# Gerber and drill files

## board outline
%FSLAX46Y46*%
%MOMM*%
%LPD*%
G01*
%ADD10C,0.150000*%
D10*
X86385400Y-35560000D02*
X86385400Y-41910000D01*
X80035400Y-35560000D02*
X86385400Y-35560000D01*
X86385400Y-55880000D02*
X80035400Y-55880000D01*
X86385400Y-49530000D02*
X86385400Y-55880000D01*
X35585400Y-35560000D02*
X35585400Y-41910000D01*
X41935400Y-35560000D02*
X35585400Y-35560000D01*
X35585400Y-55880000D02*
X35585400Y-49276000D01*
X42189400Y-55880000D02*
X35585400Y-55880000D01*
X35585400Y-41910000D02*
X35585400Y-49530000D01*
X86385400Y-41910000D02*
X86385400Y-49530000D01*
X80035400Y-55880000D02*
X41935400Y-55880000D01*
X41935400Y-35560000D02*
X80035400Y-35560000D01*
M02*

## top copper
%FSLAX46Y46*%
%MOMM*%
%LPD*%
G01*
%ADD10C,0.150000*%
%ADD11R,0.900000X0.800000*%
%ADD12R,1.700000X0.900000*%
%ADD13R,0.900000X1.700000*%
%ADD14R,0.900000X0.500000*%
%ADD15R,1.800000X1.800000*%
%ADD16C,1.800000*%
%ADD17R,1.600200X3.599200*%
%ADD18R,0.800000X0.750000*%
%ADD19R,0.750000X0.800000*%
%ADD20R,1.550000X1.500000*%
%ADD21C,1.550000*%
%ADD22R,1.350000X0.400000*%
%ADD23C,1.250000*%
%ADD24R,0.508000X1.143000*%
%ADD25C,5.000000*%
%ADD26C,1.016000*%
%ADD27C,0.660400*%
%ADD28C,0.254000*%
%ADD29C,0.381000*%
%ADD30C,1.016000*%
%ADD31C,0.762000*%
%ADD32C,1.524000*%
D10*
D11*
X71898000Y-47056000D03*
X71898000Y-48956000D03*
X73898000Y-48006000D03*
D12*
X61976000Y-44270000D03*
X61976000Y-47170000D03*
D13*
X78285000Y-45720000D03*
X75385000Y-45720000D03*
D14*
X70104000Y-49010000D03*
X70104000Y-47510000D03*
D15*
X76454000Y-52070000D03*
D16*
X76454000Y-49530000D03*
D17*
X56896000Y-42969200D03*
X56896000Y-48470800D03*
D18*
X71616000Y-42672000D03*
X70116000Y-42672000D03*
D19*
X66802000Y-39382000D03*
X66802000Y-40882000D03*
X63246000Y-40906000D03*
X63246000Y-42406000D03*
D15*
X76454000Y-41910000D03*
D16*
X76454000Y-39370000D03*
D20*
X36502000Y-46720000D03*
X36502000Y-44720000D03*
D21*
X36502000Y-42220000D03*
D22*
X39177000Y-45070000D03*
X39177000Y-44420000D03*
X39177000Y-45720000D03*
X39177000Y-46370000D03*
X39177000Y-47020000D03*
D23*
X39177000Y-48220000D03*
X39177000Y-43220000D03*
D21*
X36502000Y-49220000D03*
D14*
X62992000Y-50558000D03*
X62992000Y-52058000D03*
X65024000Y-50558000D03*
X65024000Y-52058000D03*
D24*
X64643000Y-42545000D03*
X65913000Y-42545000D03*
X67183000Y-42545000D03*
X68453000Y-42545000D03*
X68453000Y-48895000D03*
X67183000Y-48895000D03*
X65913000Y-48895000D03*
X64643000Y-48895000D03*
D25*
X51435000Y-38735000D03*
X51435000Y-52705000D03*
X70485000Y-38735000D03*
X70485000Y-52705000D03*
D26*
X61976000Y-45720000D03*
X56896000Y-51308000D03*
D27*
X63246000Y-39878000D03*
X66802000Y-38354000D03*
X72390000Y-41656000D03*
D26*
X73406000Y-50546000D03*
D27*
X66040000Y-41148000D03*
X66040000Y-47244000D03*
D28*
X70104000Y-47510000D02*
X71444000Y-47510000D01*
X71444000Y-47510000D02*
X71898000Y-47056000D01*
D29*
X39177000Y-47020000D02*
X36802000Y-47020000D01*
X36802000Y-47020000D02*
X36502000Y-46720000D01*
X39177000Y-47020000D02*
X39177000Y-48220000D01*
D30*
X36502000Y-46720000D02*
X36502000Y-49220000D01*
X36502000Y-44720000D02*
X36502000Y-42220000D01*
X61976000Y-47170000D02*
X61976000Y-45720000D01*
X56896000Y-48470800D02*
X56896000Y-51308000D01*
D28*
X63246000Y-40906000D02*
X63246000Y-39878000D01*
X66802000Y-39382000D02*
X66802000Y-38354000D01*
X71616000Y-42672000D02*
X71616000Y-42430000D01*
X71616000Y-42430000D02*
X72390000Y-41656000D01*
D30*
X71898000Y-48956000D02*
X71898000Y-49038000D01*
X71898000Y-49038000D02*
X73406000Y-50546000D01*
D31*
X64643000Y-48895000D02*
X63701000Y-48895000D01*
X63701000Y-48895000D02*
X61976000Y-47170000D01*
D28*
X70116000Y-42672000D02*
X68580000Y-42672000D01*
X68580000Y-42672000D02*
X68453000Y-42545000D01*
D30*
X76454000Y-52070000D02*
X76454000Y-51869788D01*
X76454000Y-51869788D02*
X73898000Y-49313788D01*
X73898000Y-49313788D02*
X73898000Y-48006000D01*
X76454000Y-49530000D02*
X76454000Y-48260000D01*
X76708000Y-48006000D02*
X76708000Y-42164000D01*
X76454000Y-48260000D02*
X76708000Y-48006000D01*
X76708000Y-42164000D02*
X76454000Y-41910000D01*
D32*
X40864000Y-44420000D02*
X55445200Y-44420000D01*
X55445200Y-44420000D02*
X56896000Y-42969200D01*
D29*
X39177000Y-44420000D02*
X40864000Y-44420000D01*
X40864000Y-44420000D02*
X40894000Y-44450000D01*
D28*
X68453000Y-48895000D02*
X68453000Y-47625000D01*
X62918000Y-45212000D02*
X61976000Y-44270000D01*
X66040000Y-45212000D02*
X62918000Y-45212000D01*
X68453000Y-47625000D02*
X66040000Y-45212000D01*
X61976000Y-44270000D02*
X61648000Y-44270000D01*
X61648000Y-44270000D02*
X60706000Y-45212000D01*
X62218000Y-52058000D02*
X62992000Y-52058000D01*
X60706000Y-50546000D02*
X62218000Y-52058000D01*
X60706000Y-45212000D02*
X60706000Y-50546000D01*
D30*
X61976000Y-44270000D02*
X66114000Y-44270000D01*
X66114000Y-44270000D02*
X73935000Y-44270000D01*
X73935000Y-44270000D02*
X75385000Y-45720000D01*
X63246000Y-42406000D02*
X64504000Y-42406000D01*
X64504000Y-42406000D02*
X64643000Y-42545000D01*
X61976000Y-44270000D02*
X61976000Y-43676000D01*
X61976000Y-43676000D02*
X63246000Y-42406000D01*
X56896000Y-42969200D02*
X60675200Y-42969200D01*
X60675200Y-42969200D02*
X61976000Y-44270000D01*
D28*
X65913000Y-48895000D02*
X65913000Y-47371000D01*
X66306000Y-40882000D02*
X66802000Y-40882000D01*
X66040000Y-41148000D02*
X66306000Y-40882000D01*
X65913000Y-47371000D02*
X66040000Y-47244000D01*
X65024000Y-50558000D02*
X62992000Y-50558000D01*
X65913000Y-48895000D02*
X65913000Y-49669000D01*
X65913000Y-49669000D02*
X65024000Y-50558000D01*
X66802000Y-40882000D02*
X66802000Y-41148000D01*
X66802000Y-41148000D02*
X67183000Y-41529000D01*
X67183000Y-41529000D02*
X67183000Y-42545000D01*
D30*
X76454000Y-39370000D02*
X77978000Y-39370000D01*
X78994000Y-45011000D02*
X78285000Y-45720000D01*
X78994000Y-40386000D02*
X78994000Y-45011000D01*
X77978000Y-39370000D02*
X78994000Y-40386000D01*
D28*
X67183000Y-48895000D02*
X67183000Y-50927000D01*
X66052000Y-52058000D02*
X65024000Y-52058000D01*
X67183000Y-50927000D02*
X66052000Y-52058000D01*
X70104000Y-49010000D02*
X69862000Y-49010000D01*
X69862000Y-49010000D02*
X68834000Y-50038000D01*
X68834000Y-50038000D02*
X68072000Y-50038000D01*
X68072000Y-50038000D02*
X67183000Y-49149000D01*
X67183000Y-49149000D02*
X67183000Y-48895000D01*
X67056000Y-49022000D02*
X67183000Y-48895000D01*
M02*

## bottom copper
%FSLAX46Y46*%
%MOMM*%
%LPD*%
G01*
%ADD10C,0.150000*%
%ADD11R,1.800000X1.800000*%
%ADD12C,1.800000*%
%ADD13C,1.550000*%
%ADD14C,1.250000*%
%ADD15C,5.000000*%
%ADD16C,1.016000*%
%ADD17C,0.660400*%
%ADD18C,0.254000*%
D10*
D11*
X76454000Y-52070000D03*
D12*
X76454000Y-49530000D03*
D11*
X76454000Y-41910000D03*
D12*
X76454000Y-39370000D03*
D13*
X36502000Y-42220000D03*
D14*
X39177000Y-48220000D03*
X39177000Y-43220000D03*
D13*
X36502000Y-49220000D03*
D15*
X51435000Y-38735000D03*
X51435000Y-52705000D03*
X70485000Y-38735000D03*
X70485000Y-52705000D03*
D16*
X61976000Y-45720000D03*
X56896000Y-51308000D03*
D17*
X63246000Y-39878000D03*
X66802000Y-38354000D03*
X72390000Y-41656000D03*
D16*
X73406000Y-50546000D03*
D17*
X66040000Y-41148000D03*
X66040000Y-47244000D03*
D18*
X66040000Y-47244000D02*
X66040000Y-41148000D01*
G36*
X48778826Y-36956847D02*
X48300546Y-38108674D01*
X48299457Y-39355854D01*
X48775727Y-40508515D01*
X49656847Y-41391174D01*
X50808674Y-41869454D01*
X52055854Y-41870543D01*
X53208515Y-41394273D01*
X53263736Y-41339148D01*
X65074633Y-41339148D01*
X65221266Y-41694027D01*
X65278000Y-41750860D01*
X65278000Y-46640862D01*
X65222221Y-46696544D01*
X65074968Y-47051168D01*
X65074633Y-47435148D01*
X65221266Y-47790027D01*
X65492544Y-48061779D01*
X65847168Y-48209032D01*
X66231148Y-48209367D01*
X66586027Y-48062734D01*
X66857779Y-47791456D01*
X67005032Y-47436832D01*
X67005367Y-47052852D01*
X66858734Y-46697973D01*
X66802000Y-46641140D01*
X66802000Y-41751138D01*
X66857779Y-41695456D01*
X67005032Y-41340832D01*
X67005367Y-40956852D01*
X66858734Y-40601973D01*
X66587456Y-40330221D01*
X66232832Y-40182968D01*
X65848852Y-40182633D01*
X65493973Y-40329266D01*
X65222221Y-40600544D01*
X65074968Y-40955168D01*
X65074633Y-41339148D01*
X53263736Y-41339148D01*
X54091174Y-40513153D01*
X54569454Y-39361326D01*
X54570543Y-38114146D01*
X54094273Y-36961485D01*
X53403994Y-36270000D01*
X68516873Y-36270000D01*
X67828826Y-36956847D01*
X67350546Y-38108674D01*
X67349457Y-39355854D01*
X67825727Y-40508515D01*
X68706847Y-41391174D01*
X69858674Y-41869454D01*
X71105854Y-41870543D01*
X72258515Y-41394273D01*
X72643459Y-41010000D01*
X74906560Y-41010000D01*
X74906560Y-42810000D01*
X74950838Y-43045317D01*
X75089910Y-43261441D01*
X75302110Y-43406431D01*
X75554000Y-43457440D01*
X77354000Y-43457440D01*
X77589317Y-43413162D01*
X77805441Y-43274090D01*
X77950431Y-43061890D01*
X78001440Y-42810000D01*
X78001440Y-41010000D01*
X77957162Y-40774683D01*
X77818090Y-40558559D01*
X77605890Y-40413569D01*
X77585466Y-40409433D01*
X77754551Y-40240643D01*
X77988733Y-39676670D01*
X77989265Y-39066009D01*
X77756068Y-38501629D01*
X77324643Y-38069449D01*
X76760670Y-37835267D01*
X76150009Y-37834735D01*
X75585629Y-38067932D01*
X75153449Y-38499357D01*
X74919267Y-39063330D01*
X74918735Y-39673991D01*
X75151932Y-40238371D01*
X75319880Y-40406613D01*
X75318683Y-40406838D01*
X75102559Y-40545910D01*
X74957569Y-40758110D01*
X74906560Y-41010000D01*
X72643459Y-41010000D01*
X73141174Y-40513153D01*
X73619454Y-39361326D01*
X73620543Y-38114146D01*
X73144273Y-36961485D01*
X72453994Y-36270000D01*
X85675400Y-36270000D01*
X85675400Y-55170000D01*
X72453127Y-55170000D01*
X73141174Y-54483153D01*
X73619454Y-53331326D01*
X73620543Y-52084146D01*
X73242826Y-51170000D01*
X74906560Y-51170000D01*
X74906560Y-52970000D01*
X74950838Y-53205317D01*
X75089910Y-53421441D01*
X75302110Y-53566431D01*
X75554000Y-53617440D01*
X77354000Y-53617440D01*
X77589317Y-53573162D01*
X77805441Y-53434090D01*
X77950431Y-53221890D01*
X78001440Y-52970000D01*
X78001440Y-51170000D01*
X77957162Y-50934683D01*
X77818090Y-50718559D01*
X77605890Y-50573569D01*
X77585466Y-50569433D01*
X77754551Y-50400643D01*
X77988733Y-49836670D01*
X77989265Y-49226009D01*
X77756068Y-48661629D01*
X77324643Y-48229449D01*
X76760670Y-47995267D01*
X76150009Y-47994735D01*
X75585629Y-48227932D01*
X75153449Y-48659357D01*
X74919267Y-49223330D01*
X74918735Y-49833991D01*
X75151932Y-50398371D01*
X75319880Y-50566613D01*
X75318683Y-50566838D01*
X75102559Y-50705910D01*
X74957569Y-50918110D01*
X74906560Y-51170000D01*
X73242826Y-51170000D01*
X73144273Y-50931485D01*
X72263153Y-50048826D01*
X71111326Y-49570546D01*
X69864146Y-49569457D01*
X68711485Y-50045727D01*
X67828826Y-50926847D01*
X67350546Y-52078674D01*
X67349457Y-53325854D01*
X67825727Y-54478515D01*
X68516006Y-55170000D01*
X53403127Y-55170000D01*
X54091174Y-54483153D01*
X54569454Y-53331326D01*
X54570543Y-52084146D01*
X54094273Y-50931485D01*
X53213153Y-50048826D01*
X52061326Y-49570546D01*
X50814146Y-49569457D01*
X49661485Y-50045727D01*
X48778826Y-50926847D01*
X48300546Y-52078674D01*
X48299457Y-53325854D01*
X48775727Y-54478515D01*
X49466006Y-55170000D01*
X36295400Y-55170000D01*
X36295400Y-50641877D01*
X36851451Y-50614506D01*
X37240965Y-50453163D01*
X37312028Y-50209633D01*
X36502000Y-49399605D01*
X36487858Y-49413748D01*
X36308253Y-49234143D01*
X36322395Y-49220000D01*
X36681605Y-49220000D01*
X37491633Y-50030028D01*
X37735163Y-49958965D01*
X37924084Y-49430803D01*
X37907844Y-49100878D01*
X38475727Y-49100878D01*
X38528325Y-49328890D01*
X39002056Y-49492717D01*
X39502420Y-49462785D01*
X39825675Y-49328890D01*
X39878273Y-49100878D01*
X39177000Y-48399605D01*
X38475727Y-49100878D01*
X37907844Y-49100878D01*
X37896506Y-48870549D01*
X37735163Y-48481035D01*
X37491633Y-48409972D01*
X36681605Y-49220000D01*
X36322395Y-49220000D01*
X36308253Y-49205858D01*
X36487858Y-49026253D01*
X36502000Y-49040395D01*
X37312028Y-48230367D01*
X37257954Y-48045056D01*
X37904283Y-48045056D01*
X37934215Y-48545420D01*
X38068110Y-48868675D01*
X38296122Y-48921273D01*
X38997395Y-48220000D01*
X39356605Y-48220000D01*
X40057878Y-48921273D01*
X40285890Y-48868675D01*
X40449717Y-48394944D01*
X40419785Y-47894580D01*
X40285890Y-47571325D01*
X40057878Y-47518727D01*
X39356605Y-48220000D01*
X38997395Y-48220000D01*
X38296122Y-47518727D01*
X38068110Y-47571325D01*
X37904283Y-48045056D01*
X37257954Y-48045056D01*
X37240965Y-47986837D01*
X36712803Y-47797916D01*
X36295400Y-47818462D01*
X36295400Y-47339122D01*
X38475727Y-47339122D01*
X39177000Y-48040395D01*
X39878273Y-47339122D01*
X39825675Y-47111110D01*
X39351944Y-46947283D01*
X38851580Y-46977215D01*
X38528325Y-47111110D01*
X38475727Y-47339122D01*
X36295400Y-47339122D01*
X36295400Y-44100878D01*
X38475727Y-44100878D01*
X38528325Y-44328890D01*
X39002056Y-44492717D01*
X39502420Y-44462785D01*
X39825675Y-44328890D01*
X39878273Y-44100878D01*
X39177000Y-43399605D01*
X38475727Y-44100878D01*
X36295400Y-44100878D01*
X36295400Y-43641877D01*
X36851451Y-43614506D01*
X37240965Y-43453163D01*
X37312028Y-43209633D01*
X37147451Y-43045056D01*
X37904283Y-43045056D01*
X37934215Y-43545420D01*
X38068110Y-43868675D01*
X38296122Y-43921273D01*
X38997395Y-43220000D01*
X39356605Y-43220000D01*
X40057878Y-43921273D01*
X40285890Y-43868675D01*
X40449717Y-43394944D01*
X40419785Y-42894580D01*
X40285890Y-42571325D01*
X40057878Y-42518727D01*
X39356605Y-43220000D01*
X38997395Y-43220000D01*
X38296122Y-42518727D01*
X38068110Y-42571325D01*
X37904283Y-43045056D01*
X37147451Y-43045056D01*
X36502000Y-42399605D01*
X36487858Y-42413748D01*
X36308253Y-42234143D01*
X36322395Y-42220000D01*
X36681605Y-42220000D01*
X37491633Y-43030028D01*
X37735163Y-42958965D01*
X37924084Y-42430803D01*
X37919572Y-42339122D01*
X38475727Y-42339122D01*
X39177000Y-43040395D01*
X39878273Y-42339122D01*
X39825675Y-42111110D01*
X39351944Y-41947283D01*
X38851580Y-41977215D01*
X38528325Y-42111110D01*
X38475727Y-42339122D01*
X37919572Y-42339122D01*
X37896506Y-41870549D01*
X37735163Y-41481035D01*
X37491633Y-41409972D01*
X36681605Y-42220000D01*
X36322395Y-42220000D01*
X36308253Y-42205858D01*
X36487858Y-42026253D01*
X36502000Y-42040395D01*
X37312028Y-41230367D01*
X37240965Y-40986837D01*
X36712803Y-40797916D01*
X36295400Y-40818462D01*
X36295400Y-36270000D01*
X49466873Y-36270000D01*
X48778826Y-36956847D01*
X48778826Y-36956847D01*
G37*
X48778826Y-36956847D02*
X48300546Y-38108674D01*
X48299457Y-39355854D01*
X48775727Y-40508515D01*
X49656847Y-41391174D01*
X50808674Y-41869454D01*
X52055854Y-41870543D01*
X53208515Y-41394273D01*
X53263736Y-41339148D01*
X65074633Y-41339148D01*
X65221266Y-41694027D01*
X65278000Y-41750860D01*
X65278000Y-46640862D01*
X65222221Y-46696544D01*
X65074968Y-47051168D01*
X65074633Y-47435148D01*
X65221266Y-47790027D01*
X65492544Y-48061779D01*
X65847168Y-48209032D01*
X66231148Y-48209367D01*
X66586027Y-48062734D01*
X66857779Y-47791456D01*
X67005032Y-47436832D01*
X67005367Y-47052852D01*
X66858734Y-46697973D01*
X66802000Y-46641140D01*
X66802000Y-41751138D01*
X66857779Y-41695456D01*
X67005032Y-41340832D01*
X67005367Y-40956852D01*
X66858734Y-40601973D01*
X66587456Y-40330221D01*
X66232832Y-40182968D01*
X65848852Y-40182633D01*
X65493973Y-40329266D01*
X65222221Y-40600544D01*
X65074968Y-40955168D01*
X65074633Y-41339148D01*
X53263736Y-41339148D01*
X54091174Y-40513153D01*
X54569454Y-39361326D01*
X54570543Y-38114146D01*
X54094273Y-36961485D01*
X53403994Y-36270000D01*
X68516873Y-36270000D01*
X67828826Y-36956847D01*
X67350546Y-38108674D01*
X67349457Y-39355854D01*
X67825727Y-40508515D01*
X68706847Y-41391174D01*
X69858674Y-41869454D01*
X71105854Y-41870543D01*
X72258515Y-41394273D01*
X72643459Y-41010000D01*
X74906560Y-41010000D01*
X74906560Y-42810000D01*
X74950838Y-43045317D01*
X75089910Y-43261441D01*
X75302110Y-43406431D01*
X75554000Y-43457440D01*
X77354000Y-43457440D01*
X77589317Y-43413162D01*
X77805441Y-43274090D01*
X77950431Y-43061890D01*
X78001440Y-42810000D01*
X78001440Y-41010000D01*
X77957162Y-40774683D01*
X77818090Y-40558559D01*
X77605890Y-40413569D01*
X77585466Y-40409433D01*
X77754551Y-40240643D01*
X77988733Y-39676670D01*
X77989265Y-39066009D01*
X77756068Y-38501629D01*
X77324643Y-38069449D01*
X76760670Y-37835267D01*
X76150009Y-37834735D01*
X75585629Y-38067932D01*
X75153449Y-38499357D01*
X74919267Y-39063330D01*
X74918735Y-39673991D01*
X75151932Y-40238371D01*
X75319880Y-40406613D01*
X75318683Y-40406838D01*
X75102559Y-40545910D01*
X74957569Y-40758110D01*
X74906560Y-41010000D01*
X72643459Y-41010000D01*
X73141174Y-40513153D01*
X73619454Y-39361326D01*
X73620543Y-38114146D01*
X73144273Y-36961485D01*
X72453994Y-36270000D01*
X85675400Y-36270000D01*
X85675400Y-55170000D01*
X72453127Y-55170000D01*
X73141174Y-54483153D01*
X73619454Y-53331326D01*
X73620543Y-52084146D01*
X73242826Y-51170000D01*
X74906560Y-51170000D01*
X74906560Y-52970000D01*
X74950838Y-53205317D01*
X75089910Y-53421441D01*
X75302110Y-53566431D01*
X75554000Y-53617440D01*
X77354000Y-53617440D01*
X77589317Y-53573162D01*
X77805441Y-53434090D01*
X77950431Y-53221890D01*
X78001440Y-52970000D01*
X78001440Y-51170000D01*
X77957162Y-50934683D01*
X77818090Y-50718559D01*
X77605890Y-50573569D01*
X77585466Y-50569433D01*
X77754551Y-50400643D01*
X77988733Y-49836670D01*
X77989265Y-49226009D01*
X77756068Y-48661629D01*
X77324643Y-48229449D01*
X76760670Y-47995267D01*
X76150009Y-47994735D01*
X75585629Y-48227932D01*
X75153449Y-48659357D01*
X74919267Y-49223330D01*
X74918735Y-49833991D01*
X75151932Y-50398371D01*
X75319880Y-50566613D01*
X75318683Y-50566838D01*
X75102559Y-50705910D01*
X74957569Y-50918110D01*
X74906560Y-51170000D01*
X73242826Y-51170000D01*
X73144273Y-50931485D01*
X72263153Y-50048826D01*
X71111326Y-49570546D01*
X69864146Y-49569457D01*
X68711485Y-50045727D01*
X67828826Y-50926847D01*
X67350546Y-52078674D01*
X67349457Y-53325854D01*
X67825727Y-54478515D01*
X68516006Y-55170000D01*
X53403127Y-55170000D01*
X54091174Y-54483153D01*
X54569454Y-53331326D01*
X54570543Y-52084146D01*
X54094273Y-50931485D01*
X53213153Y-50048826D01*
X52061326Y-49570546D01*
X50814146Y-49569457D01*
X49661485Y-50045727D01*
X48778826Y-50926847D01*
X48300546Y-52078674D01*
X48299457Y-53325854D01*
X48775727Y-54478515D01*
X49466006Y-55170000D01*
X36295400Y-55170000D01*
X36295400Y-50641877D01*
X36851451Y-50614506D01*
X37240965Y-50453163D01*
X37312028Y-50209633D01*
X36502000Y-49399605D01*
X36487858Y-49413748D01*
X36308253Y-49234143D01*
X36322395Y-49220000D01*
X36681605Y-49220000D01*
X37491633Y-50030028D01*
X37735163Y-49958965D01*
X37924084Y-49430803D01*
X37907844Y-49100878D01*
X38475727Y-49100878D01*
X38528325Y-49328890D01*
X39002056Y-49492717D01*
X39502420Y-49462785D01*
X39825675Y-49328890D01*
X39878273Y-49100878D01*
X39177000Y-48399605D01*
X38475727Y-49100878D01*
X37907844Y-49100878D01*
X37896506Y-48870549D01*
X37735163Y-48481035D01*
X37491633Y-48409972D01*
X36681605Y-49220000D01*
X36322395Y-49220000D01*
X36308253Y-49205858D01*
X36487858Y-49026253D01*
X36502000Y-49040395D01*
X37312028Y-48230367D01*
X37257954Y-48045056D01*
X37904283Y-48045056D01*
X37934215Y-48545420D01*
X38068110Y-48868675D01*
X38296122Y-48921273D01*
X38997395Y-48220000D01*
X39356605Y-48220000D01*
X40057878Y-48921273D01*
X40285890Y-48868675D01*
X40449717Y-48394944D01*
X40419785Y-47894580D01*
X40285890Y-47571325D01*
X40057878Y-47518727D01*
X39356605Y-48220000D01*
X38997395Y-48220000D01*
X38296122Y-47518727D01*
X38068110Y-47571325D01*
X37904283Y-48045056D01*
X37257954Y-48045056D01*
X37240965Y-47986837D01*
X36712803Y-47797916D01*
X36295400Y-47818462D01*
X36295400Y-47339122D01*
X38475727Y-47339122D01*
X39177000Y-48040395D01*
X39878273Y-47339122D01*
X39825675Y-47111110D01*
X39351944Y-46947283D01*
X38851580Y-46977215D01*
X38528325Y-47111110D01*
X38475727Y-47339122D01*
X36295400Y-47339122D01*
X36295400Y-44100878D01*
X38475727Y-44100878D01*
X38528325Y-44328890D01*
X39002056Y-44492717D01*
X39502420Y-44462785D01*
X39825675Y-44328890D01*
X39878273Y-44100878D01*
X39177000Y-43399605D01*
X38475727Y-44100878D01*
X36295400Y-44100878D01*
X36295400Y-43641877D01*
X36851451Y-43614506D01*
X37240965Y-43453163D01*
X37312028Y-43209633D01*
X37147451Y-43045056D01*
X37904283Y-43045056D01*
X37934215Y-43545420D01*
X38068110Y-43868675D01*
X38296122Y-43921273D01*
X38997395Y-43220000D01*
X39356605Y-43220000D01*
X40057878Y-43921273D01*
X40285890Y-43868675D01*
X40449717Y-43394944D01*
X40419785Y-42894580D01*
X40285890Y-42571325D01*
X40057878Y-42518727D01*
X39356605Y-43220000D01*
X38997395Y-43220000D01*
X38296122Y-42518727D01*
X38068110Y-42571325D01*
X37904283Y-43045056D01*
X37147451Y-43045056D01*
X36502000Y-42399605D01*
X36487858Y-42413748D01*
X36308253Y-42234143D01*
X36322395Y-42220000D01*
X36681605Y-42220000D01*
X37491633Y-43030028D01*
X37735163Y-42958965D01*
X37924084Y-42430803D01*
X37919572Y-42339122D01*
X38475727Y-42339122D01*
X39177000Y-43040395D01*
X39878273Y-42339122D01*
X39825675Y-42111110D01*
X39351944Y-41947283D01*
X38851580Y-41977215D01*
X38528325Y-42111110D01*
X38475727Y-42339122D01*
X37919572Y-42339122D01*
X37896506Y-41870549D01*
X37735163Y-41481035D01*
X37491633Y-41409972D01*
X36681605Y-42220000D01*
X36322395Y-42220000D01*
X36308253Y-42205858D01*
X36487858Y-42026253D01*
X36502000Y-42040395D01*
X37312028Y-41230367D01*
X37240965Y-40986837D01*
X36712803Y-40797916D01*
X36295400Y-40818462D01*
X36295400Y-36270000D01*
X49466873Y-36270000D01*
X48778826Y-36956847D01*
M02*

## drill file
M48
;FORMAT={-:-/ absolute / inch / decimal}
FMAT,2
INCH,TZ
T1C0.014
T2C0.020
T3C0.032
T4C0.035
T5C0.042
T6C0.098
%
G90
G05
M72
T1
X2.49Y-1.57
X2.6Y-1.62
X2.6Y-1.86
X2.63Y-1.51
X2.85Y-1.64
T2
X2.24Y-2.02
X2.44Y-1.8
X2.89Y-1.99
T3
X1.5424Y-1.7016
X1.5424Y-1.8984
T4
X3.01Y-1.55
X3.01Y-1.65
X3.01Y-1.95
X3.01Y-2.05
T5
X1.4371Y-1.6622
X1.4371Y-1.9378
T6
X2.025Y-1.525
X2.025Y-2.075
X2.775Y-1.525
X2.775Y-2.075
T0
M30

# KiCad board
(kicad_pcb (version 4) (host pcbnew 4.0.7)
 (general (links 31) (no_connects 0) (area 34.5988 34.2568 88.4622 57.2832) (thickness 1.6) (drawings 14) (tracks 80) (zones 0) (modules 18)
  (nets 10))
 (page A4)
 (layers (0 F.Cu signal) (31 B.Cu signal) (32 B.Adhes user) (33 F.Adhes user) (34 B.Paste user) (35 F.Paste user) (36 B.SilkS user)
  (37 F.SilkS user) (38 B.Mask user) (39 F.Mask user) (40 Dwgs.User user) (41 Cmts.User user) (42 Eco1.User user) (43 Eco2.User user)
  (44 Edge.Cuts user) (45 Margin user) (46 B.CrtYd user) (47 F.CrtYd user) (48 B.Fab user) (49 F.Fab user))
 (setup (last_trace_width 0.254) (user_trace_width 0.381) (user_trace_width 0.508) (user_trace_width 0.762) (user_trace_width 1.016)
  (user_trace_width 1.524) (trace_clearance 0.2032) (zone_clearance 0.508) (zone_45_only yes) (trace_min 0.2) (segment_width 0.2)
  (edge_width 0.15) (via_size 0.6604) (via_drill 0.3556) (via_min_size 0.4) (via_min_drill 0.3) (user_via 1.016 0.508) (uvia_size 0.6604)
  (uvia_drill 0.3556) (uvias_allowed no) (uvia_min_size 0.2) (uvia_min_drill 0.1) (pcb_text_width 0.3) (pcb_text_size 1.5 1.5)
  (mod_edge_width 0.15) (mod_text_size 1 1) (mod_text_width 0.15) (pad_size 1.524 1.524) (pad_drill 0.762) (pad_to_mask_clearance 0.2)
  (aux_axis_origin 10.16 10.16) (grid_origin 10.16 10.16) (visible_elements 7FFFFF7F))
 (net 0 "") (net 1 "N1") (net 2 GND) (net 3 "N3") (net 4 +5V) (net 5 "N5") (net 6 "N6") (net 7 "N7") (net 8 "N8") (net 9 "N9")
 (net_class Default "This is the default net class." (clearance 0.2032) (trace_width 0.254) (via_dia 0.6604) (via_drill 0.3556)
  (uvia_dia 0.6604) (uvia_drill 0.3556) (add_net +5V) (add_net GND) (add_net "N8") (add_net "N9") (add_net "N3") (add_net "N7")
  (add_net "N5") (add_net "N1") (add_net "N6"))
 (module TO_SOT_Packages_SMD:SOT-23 (layer F.Cu) (at 72.898 48.006)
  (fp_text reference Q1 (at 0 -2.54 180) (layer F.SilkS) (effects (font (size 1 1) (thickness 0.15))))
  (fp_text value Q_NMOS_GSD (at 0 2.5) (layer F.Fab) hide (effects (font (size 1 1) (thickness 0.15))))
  (pad 1 smd rect (at -1 -0.95) (size 0.9 0.8) (layers F.Cu F.Paste F.Mask) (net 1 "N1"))
  (pad 2 smd rect (at -1 0.95) (size 0.9 0.8) (layers F.Cu F.Paste F.Mask) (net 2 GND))
  (pad 3 smd rect (at 1 0) (size 0.9 0.8) (layers F.Cu F.Paste F.Mask) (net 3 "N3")))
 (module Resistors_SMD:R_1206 (layer F.Cu) (at 61.976 45.72 270)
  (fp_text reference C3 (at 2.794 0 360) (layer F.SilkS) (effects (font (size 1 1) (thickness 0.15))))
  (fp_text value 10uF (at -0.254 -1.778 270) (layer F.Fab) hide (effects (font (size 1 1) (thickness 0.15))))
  (pad 1 smd rect (at -1.45 0 270) (size 0.9 1.7) (layers F.Cu F.Paste F.Mask) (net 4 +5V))
  (pad 2 smd rect (at 1.45 0 270) (size 0.9 1.7) (layers F.Cu F.Paste F.Mask) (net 2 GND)))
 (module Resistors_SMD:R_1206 (layer F.Cu) (at 76.835 45.72 180)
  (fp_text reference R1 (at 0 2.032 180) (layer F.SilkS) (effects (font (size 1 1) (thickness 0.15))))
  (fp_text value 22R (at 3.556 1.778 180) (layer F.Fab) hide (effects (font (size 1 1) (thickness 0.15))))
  (pad 1 smd rect (at -1.45 0 180) (size 0.9 1.7) (layers F.Cu F.Paste F.Mask) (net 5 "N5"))
  (pad 2 smd rect (at 1.45 0 180) (size 0.9 1.7) (layers F.Cu F.Paste F.Mask) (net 4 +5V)))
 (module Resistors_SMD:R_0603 (layer F.Cu) (at 70.104 48.26 90)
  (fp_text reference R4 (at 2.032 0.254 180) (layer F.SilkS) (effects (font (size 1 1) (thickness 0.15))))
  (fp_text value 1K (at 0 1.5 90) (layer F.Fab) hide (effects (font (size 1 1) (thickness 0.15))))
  (pad 1 smd rect (at -0.75 0 90) (size 0.5 0.9) (layers F.Cu F.Paste F.Mask) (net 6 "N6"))
  (pad 2 smd rect (at 0.75 0 90) (size 0.5 0.9) (layers F.Cu F.Paste F.Mask) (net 1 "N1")))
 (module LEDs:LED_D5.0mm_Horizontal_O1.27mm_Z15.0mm (layer F.Cu) (at 76.454 52.07 90)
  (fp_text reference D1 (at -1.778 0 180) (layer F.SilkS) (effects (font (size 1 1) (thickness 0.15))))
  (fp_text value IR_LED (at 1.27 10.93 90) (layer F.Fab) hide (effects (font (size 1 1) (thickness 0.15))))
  (pad 1 thru_hole rect (at 0 0 90) (size 1.8 1.8) (drill 0.9) (layers *.Cu *.Mask) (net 3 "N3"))
  (pad 2 thru_hole circle (at 2.54 0 90) (size 1.8 1.8) (drill 0.9) (layers *.Cu *.Mask) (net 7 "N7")))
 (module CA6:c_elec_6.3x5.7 (layer F.Cu) (at 56.896 45.72 90)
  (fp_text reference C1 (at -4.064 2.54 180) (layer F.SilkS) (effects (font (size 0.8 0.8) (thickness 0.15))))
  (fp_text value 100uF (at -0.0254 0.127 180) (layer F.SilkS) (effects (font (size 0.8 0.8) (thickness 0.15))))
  (pad 1 smd rect (at 2.7508 0 90) (size 3.5992 1.6002) (layers F.Cu F.Paste F.Mask) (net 4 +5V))
  (pad 2 smd rect (at -2.7508 0 90) (size 3.5992 1.6002) (layers F.Cu F.Paste F.Mask) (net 2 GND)))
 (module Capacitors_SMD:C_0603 (layer F.Cu) (at 70.866 42.672)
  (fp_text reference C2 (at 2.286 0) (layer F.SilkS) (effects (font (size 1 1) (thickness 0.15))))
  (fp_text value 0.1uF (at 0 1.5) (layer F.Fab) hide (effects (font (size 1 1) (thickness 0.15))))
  (pad 2 smd rect (at 0.75 0) (size 0.8 0.75) (layers F.Cu F.Paste F.Mask) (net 2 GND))
  (pad 1 smd rect (at -0.75 0) (size 0.8 0.75) (layers F.Cu F.Paste F.Mask) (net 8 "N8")))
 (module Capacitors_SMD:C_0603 (layer F.Cu) (at 66.802 40.132 90)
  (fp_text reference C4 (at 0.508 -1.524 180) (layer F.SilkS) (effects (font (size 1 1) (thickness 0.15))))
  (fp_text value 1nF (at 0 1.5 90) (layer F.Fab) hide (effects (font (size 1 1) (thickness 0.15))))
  (pad 2 smd rect (at 0.75 0 90) (size 0.8 0.75) (layers F.Cu F.Paste F.Mask) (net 2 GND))
  (pad 1 smd rect (at -0.75 0 90) (size 0.8 0.75) (layers F.Cu F.Paste F.Mask) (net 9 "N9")))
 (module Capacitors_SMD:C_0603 (layer F.Cu) (at 63.246 41.656 90)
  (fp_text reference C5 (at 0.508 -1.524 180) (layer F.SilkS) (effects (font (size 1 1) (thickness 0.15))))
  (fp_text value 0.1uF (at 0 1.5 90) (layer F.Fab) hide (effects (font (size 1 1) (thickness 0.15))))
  (pad 2 smd rect (at 0.75 0 90) (size 0.8 0.75) (layers F.Cu F.Paste F.Mask) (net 2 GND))
  (pad 1 smd rect (at -0.75 0 90) (size 0.8 0.75) (layers F.Cu F.Paste F.Mask) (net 4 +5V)))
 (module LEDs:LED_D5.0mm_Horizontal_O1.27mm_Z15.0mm (layer F.Cu) (at 76.454 41.91 90)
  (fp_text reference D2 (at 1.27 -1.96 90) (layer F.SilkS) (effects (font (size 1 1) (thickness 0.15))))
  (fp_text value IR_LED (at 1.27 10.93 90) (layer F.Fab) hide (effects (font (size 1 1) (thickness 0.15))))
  (pad 1 thru_hole rect (at 0 0 90) (size 1.8 1.8) (drill 0.9) (layers *.Cu *.Mask) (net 7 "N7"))
  (pad 2 thru_hole circle (at 2.54 0 90) (size 1.8 1.8) (drill 0.9) (layers *.Cu *.Mask) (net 5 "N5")))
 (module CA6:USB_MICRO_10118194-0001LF (layer F.Cu) (at 35.052 45.72 270)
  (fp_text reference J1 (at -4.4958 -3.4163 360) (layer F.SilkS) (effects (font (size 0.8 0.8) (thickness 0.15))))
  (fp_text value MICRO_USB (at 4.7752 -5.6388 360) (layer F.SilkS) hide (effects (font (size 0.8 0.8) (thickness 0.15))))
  (pad 5 smd rect (at 1 -1.45 270) (size 1.5 1.55) (layers F.Cu F.Paste F.Mask) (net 2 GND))
  (pad 5 smd rect (at -1 -1.45 270) (size 1.5 1.55) (layers F.Cu F.Paste F.Mask) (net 2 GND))
  (pad 5 thru_hole circle (at -3.5 -1.45 270) (size 1.55 1.55) (drill 1.0668) (layers *.Cu *.Mask F.SilkS) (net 2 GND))
  (pad 2 smd rect (at -0.65 -4.125 270) (size 0.4 1.35) (layers F.Cu F.Paste F.Mask))
  (pad 1 smd rect (at -1.3 -4.125 270) (size 0.4 1.35) (layers F.Cu F.Paste F.Mask) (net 4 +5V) (clearance 0.19))
  (pad 3 smd rect (at 0 -4.125 270) (size 0.4 1.35) (layers F.Cu F.Paste F.Mask))
  (pad 4 smd rect (at 0.65 -4.125 270) (size 0.4 1.35) (layers F.Cu F.Paste F.Mask))
  (pad 5 smd rect (at 1.3 -4.125 270) (size 0.4 1.35) (layers F.Cu F.Paste F.Mask) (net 2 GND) (clearance 0.19))
  (pad 5 thru_hole circle (at 2.5 -4.125 270) (size 1.25 1.25) (drill 0.8128) (layers *.Cu *.Mask F.SilkS) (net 2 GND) (clearance 0.19))
  (pad 5 thru_hole circle (at -2.5 -4.125 270) (size 1.25 1.25) (drill 0.8128) (layers *.Cu *.Mask F.SilkS) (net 2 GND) (clearance 0.19))
  (pad 5 thru_hole circle (at 3.5 -1.45 270) (size 1.55 1.55) (drill 1.0668) (layers *.Cu *.Mask F.SilkS) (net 2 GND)))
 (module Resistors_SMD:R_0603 (layer F.Cu) (at 62.992 51.308 270)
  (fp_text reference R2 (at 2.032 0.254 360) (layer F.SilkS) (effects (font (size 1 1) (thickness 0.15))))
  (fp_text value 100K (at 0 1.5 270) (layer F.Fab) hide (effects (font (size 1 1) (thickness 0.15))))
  (pad 1 smd rect (at -0.75 0 270) (size 0.5 0.9) (layers F.Cu F.Paste F.Mask) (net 9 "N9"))
  (pad 2 smd rect (at 0.75 0 270) (size 0.5 0.9) (layers F.Cu F.Paste F.Mask) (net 4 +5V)))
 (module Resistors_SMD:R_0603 (layer F.Cu) (at 65.024 51.308 270)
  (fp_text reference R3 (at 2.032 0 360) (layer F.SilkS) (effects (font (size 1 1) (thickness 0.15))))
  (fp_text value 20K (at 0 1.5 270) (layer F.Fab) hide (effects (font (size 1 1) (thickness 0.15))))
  (pad 1 smd rect (at -0.75 0 270) (size 0.5 0.9) (layers F.Cu F.Paste F.Mask) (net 9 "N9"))
  (pad 2 smd rect (at 0.75 0 270) (size 0.5 0.9) (layers F.Cu F.Paste F.Mask) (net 6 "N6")))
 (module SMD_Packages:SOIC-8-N (layer F.Cu) (at 66.548 45.72)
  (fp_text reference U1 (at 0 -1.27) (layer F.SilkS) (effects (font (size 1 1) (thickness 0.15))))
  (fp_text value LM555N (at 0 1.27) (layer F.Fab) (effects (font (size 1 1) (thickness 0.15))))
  (pad 8 smd rect (at -1.905 -3.175) (size 0.508 1.143) (layers F.Cu F.Paste F.Mask) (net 4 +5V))
  (pad 7 smd rect (at -0.635 -3.175) (size 0.508 1.143) (layers F.Cu F.Paste F.Mask))
  (pad 6 smd rect (at 0.635 -3.175) (size 0.508 1.143) (layers F.Cu F.Paste F.Mask) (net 9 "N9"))
  (pad 5 smd rect (at 1.905 -3.175) (size 0.508 1.143) (layers F.Cu F.Paste F.Mask) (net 8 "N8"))
  (pad 4 smd rect (at 1.905 3.175) (size 0.508 1.143) (layers F.Cu F.Paste F.Mask) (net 4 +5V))
  (pad 3 smd rect (at 0.635 3.175) (size 0.508 1.143) (layers F.Cu F.Paste F.Mask) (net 6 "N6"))
  (pad 2 smd rect (at -0.635 3.175) (size 0.508 1.143) (layers F.Cu F.Paste F.Mask) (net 9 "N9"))
  (pad 1 smd rect (at -1.905 3.175) (size 0.508 1.143) (layers F.Cu F.Paste F.Mask) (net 2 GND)))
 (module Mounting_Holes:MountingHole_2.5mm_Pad (layer F.Cu) (at 51.435 38.735)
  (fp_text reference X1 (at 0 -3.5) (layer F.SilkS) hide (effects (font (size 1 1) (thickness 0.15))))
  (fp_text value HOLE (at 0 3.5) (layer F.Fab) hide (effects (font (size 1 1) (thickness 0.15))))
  (pad 1 thru_hole circle (at 0 0) (size 5 5) (drill 2.5) (layers *.Cu *.Mask)))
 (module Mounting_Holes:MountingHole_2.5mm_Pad (layer F.Cu) (at 51.435 52.705)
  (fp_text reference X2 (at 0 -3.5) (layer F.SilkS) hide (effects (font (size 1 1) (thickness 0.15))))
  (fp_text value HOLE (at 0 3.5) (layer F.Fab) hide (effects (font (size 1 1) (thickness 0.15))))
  (pad 1 thru_hole circle (at 0 0) (size 5 5) (drill 2.5) (layers *.Cu *.Mask)))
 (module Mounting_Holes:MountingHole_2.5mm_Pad (layer F.Cu) (at 70.485 38.735)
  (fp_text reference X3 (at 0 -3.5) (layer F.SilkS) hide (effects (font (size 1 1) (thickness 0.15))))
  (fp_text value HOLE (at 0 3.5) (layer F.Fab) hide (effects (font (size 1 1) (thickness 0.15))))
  (pad 1 thru_hole circle (at 0 0) (size 5 5) (drill 2.5) (layers *.Cu *.Mask)))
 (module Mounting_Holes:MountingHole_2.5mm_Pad (layer F.Cu) (at 70.485 52.705)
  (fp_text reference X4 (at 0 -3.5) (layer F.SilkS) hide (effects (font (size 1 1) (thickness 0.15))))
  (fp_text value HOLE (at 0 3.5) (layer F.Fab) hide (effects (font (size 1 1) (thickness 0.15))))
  (pad 1 thru_hole circle (at 0 0) (size 5 5) (drill 2.5) (layers *.Cu *.Mask)))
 (gr_line (start 86.3854 35.56) (end 86.3854 41.91) (angle 90) (layer Edge.Cuts) (width 0.15))
 (gr_line (start 80.0354 35.56) (end 86.3854 35.56) (angle 90) (layer Edge.Cuts) (width 0.15))
 (gr_line (start 86.3854 55.88) (end 80.0354 55.88) (angle 90) (layer Edge.Cuts) (width 0.15))
 (gr_line (start 86.3854 49.53) (end 86.3854 55.88) (angle 90) (layer Edge.Cuts) (width 0.15))
 (gr_line (start 35.5854 35.56) (end 35.5854 41.91) (angle 90) (layer Edge.Cuts) (width 0.15))
 (gr_line (start 41.9354 35.56) (end 35.5854 35.56) (angle 90) (layer Edge.Cuts) (width 0.15))
 (gr_line (start 35.5854 55.88) (end 35.5854 49.276) (angle 90) (layer Edge.Cuts) (width 0.15))
 (gr_line (start 42.1894 55.88) (end 35.5854 55.88) (angle 90) (layer Edge.Cuts) (width 0.15))
 (gr_line (start 35.5854 41.91) (end 35.5854 49.53) (angle 90) (layer Edge.Cuts) (width 0.15))
 (gr_line (start 86.3854 41.91) (end 86.3854 49.53) (angle 90) (layer Edge.Cuts) (width 0.15))
 (gr_line (start 80.0354 55.88) (end 41.9354 55.88) (angle 90) (layer Edge.Cuts) (width 0.15))
 (gr_line (start 41.9354 35.56) (end 80.0354 35.56) (angle 90) (layer Edge.Cuts) (width 0.15))
 (segment (start 70.104 47.51) (end 71.444 47.51) (width 0.254) (layer F.Cu) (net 1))
 (segment (start 71.444 47.51) (end 71.898 47.056) (width 0.254) (layer F.Cu) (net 1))
 (segment (start 39.177 47.02) (end 36.802 47.02) (width 0.381) (layer F.Cu) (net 2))
 (segment (start 36.802 47.02) (end 36.502 46.72) (width 0.381) (layer F.Cu) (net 2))
 (segment (start 39.177 47.02) (end 39.177 48.22) (width 0.381) (layer F.Cu) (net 2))
 (segment (start 36.502 46.72) (end 36.502 49.22) (width 1.016) (layer F.Cu) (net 2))
 (segment (start 36.502 44.72) (end 36.502 42.22) (width 1.016) (layer F.Cu) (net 2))
 (segment (start 61.976 47.17) (end 61.976 45.72) (width 1.016) (layer F.Cu) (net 2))
 (via (at 61.976 45.72) (size 1.016) (drill 0.508) (layers F.Cu B.Cu) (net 2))
 (segment (start 56.896 48.4708) (end 56.896 51.308) (width 1.016) (layer F.Cu) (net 2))
 (via (at 56.896 51.308) (size 1.016) (drill 0.508) (layers F.Cu B.Cu) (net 2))
 (segment (start 63.246 40.906) (end 63.246 39.878) (width 0.254) (layer F.Cu) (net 2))
 (via (at 63.246 39.878) (size 0.6604) (drill 0.3556) (layers F.Cu B.Cu) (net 2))
 (segment (start 66.802 39.382) (end 66.802 38.354) (width 0.254) (layer F.Cu) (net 2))
 (via (at 66.802 38.354) (size 0.6604) (drill 0.3556) (layers F.Cu B.Cu) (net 2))
 (segment (start 71.616 42.672) (end 71.616 42.43) (width 0.254) (layer F.Cu) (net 2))
 (segment (start 71.616 42.43) (end 72.39 41.656) (width 0.254) (layer F.Cu) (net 2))
 (via (at 72.39 41.656) (size 0.6604) (drill 0.3556) (layers F.Cu B.Cu) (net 2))
 (segment (start 71.898 48.956) (end 71.898 49.038) (width 1.016) (layer F.Cu) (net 2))
 (segment (start 71.898 49.038) (end 73.406 50.546) (width 1.016) (layer F.Cu) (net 2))
 (via (at 73.406 50.546) (size 1.016) (drill 0.508) (layers F.Cu B.Cu) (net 2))
 (segment (start 64.643 48.895) (end 63.701 48.895) (width 0.762) (layer F.Cu) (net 2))
 (segment (start 63.701 48.895) (end 61.976 47.17) (width 0.762) (layer F.Cu) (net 2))
 (segment (start 70.116 42.672) (end 68.58 42.672) (width 0.254) (layer F.Cu) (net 8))
 (segment (start 68.58 42.672) (end 68.453 42.545) (width 0.254) (layer F.Cu) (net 8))
 (segment (start 76.454 52.07) (end 76.454 51.869788) (width 1.016) (layer F.Cu) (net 3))
 (segment (start 76.454 51.869788) (end 73.898 49.313788) (width 1.016) (layer F.Cu) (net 3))
 (segment (start 73.898 49.313788) (end 73.898 48.006) (width 1.016) (layer F.Cu) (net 3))
 (segment (start 76.454 49.53) (end 76.454 48.26) (width 1.016) (layer F.Cu) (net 7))
 (segment (start 76.708 48.006) (end 76.708 42.164) (width 1.016) (layer F.Cu) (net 7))
 (segment (start 76.454 48.26) (end 76.708 48.006) (width 1.016) (layer F.Cu) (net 7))
 (segment (start 76.708 42.164) (end 76.454 41.91) (width 1.016) (layer F.Cu) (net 7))
 (segment (start 40.864 44.42) (end 55.4452 44.42) (width 1.524) (layer F.Cu) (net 4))
 (segment (start 55.4452 44.42) (end 56.896 42.9692) (width 1.524) (layer F.Cu) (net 4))
 (segment (start 39.177 44.42) (end 40.864 44.42) (width 0.381) (layer F.Cu) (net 4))
 (segment (start 40.864 44.42) (end 40.894 44.45) (width 0.381) (layer F.Cu) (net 4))
 (segment (start 68.453 48.895) (end 68.453 47.625) (width 0.254) (layer F.Cu) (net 4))
 (segment (start 62.918 45.212) (end 61.976 44.27) (width 0.254) (layer F.Cu) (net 4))
 (segment (start 66.04 45.212) (end 62.918 45.212) (width 0.254) (layer F.Cu) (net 4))
 (segment (start 68.453 47.625) (end 66.04 45.212) (width 0.254) (layer F.Cu) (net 4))
 (segment (start 61.976 44.27) (end 61.648 44.27) (width 0.254) (layer F.Cu) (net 4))
 (segment (start 61.648 44.27) (end 60.706 45.212) (width 0.254) (layer F.Cu) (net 4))
 (segment (start 62.218 52.058) (end 62.992 52.058) (width 0.254) (layer F.Cu) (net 4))
 (segment (start 60.706 50.546) (end 62.218 52.058) (width 0.254) (layer F.Cu) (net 4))
 (segment (start 60.706 45.212) (end 60.706 50.546) (width 0.254) (layer F.Cu) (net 4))
 (segment (start 61.976 44.27) (end 66.114 44.27) (width 1.016) (layer F.Cu) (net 4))
 (segment (start 66.114 44.27) (end 73.935 44.27) (width 1.016) (layer F.Cu) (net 4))
 (segment (start 73.935 44.27) (end 75.385 45.72) (width 1.016) (layer F.Cu) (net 4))
 (segment (start 63.246 42.406) (end 64.504 42.406) (width 1.016) (layer F.Cu) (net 4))
 (segment (start 64.504 42.406) (end 64.643 42.545) (width 1.016) (layer F.Cu) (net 4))
 (segment (start 61.976 44.27) (end 61.976 43.676) (width 1.016) (layer F.Cu) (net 4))
 (segment (start 61.976 43.676) (end 63.246 42.406) (width 1.016) (layer F.Cu) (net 4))
 (segment (start 56.896 42.9692) (end 60.6752 42.9692) (width 1.016) (layer F.Cu) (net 4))
 (segment (start 60.6752 42.9692) (end 61.976 44.27) (width 1.016) (layer F.Cu) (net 4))
 (segment (start 65.913 48.895) (end 65.913 47.371) (width 0.254) (layer F.Cu) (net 9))
 (segment (start 66.306 40.882) (end 66.802 40.882) (width 0.254) (layer F.Cu) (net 9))
 (segment (start 66.04 41.148) (end 66.306 40.882) (width 0.254) (layer F.Cu) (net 9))
 (via (at 66.04 41.148) (size 0.6604) (drill 0.3556) (layers F.Cu B.Cu) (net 9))
 (segment (start 66.04 47.244) (end 66.04 41.148) (width 0.254) (layer B.Cu) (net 9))
 (via (at 66.04 47.244) (size 0.6604) (drill 0.3556) (layers F.Cu B.Cu) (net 9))
 (segment (start 65.913 47.371) (end 66.04 47.244) (width 0.254) (layer F.Cu) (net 9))
 (segment (start 65.024 50.558) (end 62.992 50.558) (width 0.254) (layer F.Cu) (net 9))
 (segment (start 65.913 48.895) (end 65.913 49.669) (width 0.254) (layer F.Cu) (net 9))
 (segment (start 65.913 49.669) (end 65.024 50.558) (width 0.254) (layer F.Cu) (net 9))
 (segment (start 66.802 40.882) (end 66.802 41.148) (width 0.254) (layer F.Cu) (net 9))
 (segment (start 66.802 41.148) (end 67.183 41.529) (width 0.254) (layer F.Cu) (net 9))
 (segment (start 67.183 41.529) (end 67.183 42.545) (width 0.254) (layer F.Cu) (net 9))
 (segment (start 76.454 39.37) (end 77.978 39.37) (width 1.016) (layer F.Cu) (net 5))
 (segment (start 78.994 45.011) (end 78.285 45.72) (width 1.016) (layer F.Cu) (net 5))
 (segment (start 78.994 40.386) (end 78.994 45.011) (width 1.016) (layer F.Cu) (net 5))
 (segment (start 77.978 39.37) (end 78.994 40.386) (width 1.016) (layer F.Cu) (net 5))
 (segment (start 67.183 48.895) (end 67.183 50.927) (width 0.254) (layer F.Cu) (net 6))
 (segment (start 66.052 52.058) (end 65.024 52.058) (width 0.254) (layer F.Cu) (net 6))
 (segment (start 67.183 50.927) (end 66.052 52.058) (width 0.254) (layer F.Cu) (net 6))
 (segment (start 70.104 49.01) (end 69.862 49.01) (width 0.254) (layer F.Cu) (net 6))
 (segment (start 69.862 49.01) (end 68.834 50.038) (width 0.254) (layer F.Cu) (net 6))
 (segment (start 68.834 50.038) (end 68.072 50.038) (width 0.254) (layer F.Cu) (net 6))
 (segment (start 68.072 50.038) (end 67.183 49.149) (width 0.254) (layer F.Cu) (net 6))
 (segment (start 67.183 49.149) (end 67.183 48.895) (width 0.254) (layer F.Cu) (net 6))
 (segment (start 67.056 49.022) (end 67.183 48.895) (width 0.254) (layer F.Cu) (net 6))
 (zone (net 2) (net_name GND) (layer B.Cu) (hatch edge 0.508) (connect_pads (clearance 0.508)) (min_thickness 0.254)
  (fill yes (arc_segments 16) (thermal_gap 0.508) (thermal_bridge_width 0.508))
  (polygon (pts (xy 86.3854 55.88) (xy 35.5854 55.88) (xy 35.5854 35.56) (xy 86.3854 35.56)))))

